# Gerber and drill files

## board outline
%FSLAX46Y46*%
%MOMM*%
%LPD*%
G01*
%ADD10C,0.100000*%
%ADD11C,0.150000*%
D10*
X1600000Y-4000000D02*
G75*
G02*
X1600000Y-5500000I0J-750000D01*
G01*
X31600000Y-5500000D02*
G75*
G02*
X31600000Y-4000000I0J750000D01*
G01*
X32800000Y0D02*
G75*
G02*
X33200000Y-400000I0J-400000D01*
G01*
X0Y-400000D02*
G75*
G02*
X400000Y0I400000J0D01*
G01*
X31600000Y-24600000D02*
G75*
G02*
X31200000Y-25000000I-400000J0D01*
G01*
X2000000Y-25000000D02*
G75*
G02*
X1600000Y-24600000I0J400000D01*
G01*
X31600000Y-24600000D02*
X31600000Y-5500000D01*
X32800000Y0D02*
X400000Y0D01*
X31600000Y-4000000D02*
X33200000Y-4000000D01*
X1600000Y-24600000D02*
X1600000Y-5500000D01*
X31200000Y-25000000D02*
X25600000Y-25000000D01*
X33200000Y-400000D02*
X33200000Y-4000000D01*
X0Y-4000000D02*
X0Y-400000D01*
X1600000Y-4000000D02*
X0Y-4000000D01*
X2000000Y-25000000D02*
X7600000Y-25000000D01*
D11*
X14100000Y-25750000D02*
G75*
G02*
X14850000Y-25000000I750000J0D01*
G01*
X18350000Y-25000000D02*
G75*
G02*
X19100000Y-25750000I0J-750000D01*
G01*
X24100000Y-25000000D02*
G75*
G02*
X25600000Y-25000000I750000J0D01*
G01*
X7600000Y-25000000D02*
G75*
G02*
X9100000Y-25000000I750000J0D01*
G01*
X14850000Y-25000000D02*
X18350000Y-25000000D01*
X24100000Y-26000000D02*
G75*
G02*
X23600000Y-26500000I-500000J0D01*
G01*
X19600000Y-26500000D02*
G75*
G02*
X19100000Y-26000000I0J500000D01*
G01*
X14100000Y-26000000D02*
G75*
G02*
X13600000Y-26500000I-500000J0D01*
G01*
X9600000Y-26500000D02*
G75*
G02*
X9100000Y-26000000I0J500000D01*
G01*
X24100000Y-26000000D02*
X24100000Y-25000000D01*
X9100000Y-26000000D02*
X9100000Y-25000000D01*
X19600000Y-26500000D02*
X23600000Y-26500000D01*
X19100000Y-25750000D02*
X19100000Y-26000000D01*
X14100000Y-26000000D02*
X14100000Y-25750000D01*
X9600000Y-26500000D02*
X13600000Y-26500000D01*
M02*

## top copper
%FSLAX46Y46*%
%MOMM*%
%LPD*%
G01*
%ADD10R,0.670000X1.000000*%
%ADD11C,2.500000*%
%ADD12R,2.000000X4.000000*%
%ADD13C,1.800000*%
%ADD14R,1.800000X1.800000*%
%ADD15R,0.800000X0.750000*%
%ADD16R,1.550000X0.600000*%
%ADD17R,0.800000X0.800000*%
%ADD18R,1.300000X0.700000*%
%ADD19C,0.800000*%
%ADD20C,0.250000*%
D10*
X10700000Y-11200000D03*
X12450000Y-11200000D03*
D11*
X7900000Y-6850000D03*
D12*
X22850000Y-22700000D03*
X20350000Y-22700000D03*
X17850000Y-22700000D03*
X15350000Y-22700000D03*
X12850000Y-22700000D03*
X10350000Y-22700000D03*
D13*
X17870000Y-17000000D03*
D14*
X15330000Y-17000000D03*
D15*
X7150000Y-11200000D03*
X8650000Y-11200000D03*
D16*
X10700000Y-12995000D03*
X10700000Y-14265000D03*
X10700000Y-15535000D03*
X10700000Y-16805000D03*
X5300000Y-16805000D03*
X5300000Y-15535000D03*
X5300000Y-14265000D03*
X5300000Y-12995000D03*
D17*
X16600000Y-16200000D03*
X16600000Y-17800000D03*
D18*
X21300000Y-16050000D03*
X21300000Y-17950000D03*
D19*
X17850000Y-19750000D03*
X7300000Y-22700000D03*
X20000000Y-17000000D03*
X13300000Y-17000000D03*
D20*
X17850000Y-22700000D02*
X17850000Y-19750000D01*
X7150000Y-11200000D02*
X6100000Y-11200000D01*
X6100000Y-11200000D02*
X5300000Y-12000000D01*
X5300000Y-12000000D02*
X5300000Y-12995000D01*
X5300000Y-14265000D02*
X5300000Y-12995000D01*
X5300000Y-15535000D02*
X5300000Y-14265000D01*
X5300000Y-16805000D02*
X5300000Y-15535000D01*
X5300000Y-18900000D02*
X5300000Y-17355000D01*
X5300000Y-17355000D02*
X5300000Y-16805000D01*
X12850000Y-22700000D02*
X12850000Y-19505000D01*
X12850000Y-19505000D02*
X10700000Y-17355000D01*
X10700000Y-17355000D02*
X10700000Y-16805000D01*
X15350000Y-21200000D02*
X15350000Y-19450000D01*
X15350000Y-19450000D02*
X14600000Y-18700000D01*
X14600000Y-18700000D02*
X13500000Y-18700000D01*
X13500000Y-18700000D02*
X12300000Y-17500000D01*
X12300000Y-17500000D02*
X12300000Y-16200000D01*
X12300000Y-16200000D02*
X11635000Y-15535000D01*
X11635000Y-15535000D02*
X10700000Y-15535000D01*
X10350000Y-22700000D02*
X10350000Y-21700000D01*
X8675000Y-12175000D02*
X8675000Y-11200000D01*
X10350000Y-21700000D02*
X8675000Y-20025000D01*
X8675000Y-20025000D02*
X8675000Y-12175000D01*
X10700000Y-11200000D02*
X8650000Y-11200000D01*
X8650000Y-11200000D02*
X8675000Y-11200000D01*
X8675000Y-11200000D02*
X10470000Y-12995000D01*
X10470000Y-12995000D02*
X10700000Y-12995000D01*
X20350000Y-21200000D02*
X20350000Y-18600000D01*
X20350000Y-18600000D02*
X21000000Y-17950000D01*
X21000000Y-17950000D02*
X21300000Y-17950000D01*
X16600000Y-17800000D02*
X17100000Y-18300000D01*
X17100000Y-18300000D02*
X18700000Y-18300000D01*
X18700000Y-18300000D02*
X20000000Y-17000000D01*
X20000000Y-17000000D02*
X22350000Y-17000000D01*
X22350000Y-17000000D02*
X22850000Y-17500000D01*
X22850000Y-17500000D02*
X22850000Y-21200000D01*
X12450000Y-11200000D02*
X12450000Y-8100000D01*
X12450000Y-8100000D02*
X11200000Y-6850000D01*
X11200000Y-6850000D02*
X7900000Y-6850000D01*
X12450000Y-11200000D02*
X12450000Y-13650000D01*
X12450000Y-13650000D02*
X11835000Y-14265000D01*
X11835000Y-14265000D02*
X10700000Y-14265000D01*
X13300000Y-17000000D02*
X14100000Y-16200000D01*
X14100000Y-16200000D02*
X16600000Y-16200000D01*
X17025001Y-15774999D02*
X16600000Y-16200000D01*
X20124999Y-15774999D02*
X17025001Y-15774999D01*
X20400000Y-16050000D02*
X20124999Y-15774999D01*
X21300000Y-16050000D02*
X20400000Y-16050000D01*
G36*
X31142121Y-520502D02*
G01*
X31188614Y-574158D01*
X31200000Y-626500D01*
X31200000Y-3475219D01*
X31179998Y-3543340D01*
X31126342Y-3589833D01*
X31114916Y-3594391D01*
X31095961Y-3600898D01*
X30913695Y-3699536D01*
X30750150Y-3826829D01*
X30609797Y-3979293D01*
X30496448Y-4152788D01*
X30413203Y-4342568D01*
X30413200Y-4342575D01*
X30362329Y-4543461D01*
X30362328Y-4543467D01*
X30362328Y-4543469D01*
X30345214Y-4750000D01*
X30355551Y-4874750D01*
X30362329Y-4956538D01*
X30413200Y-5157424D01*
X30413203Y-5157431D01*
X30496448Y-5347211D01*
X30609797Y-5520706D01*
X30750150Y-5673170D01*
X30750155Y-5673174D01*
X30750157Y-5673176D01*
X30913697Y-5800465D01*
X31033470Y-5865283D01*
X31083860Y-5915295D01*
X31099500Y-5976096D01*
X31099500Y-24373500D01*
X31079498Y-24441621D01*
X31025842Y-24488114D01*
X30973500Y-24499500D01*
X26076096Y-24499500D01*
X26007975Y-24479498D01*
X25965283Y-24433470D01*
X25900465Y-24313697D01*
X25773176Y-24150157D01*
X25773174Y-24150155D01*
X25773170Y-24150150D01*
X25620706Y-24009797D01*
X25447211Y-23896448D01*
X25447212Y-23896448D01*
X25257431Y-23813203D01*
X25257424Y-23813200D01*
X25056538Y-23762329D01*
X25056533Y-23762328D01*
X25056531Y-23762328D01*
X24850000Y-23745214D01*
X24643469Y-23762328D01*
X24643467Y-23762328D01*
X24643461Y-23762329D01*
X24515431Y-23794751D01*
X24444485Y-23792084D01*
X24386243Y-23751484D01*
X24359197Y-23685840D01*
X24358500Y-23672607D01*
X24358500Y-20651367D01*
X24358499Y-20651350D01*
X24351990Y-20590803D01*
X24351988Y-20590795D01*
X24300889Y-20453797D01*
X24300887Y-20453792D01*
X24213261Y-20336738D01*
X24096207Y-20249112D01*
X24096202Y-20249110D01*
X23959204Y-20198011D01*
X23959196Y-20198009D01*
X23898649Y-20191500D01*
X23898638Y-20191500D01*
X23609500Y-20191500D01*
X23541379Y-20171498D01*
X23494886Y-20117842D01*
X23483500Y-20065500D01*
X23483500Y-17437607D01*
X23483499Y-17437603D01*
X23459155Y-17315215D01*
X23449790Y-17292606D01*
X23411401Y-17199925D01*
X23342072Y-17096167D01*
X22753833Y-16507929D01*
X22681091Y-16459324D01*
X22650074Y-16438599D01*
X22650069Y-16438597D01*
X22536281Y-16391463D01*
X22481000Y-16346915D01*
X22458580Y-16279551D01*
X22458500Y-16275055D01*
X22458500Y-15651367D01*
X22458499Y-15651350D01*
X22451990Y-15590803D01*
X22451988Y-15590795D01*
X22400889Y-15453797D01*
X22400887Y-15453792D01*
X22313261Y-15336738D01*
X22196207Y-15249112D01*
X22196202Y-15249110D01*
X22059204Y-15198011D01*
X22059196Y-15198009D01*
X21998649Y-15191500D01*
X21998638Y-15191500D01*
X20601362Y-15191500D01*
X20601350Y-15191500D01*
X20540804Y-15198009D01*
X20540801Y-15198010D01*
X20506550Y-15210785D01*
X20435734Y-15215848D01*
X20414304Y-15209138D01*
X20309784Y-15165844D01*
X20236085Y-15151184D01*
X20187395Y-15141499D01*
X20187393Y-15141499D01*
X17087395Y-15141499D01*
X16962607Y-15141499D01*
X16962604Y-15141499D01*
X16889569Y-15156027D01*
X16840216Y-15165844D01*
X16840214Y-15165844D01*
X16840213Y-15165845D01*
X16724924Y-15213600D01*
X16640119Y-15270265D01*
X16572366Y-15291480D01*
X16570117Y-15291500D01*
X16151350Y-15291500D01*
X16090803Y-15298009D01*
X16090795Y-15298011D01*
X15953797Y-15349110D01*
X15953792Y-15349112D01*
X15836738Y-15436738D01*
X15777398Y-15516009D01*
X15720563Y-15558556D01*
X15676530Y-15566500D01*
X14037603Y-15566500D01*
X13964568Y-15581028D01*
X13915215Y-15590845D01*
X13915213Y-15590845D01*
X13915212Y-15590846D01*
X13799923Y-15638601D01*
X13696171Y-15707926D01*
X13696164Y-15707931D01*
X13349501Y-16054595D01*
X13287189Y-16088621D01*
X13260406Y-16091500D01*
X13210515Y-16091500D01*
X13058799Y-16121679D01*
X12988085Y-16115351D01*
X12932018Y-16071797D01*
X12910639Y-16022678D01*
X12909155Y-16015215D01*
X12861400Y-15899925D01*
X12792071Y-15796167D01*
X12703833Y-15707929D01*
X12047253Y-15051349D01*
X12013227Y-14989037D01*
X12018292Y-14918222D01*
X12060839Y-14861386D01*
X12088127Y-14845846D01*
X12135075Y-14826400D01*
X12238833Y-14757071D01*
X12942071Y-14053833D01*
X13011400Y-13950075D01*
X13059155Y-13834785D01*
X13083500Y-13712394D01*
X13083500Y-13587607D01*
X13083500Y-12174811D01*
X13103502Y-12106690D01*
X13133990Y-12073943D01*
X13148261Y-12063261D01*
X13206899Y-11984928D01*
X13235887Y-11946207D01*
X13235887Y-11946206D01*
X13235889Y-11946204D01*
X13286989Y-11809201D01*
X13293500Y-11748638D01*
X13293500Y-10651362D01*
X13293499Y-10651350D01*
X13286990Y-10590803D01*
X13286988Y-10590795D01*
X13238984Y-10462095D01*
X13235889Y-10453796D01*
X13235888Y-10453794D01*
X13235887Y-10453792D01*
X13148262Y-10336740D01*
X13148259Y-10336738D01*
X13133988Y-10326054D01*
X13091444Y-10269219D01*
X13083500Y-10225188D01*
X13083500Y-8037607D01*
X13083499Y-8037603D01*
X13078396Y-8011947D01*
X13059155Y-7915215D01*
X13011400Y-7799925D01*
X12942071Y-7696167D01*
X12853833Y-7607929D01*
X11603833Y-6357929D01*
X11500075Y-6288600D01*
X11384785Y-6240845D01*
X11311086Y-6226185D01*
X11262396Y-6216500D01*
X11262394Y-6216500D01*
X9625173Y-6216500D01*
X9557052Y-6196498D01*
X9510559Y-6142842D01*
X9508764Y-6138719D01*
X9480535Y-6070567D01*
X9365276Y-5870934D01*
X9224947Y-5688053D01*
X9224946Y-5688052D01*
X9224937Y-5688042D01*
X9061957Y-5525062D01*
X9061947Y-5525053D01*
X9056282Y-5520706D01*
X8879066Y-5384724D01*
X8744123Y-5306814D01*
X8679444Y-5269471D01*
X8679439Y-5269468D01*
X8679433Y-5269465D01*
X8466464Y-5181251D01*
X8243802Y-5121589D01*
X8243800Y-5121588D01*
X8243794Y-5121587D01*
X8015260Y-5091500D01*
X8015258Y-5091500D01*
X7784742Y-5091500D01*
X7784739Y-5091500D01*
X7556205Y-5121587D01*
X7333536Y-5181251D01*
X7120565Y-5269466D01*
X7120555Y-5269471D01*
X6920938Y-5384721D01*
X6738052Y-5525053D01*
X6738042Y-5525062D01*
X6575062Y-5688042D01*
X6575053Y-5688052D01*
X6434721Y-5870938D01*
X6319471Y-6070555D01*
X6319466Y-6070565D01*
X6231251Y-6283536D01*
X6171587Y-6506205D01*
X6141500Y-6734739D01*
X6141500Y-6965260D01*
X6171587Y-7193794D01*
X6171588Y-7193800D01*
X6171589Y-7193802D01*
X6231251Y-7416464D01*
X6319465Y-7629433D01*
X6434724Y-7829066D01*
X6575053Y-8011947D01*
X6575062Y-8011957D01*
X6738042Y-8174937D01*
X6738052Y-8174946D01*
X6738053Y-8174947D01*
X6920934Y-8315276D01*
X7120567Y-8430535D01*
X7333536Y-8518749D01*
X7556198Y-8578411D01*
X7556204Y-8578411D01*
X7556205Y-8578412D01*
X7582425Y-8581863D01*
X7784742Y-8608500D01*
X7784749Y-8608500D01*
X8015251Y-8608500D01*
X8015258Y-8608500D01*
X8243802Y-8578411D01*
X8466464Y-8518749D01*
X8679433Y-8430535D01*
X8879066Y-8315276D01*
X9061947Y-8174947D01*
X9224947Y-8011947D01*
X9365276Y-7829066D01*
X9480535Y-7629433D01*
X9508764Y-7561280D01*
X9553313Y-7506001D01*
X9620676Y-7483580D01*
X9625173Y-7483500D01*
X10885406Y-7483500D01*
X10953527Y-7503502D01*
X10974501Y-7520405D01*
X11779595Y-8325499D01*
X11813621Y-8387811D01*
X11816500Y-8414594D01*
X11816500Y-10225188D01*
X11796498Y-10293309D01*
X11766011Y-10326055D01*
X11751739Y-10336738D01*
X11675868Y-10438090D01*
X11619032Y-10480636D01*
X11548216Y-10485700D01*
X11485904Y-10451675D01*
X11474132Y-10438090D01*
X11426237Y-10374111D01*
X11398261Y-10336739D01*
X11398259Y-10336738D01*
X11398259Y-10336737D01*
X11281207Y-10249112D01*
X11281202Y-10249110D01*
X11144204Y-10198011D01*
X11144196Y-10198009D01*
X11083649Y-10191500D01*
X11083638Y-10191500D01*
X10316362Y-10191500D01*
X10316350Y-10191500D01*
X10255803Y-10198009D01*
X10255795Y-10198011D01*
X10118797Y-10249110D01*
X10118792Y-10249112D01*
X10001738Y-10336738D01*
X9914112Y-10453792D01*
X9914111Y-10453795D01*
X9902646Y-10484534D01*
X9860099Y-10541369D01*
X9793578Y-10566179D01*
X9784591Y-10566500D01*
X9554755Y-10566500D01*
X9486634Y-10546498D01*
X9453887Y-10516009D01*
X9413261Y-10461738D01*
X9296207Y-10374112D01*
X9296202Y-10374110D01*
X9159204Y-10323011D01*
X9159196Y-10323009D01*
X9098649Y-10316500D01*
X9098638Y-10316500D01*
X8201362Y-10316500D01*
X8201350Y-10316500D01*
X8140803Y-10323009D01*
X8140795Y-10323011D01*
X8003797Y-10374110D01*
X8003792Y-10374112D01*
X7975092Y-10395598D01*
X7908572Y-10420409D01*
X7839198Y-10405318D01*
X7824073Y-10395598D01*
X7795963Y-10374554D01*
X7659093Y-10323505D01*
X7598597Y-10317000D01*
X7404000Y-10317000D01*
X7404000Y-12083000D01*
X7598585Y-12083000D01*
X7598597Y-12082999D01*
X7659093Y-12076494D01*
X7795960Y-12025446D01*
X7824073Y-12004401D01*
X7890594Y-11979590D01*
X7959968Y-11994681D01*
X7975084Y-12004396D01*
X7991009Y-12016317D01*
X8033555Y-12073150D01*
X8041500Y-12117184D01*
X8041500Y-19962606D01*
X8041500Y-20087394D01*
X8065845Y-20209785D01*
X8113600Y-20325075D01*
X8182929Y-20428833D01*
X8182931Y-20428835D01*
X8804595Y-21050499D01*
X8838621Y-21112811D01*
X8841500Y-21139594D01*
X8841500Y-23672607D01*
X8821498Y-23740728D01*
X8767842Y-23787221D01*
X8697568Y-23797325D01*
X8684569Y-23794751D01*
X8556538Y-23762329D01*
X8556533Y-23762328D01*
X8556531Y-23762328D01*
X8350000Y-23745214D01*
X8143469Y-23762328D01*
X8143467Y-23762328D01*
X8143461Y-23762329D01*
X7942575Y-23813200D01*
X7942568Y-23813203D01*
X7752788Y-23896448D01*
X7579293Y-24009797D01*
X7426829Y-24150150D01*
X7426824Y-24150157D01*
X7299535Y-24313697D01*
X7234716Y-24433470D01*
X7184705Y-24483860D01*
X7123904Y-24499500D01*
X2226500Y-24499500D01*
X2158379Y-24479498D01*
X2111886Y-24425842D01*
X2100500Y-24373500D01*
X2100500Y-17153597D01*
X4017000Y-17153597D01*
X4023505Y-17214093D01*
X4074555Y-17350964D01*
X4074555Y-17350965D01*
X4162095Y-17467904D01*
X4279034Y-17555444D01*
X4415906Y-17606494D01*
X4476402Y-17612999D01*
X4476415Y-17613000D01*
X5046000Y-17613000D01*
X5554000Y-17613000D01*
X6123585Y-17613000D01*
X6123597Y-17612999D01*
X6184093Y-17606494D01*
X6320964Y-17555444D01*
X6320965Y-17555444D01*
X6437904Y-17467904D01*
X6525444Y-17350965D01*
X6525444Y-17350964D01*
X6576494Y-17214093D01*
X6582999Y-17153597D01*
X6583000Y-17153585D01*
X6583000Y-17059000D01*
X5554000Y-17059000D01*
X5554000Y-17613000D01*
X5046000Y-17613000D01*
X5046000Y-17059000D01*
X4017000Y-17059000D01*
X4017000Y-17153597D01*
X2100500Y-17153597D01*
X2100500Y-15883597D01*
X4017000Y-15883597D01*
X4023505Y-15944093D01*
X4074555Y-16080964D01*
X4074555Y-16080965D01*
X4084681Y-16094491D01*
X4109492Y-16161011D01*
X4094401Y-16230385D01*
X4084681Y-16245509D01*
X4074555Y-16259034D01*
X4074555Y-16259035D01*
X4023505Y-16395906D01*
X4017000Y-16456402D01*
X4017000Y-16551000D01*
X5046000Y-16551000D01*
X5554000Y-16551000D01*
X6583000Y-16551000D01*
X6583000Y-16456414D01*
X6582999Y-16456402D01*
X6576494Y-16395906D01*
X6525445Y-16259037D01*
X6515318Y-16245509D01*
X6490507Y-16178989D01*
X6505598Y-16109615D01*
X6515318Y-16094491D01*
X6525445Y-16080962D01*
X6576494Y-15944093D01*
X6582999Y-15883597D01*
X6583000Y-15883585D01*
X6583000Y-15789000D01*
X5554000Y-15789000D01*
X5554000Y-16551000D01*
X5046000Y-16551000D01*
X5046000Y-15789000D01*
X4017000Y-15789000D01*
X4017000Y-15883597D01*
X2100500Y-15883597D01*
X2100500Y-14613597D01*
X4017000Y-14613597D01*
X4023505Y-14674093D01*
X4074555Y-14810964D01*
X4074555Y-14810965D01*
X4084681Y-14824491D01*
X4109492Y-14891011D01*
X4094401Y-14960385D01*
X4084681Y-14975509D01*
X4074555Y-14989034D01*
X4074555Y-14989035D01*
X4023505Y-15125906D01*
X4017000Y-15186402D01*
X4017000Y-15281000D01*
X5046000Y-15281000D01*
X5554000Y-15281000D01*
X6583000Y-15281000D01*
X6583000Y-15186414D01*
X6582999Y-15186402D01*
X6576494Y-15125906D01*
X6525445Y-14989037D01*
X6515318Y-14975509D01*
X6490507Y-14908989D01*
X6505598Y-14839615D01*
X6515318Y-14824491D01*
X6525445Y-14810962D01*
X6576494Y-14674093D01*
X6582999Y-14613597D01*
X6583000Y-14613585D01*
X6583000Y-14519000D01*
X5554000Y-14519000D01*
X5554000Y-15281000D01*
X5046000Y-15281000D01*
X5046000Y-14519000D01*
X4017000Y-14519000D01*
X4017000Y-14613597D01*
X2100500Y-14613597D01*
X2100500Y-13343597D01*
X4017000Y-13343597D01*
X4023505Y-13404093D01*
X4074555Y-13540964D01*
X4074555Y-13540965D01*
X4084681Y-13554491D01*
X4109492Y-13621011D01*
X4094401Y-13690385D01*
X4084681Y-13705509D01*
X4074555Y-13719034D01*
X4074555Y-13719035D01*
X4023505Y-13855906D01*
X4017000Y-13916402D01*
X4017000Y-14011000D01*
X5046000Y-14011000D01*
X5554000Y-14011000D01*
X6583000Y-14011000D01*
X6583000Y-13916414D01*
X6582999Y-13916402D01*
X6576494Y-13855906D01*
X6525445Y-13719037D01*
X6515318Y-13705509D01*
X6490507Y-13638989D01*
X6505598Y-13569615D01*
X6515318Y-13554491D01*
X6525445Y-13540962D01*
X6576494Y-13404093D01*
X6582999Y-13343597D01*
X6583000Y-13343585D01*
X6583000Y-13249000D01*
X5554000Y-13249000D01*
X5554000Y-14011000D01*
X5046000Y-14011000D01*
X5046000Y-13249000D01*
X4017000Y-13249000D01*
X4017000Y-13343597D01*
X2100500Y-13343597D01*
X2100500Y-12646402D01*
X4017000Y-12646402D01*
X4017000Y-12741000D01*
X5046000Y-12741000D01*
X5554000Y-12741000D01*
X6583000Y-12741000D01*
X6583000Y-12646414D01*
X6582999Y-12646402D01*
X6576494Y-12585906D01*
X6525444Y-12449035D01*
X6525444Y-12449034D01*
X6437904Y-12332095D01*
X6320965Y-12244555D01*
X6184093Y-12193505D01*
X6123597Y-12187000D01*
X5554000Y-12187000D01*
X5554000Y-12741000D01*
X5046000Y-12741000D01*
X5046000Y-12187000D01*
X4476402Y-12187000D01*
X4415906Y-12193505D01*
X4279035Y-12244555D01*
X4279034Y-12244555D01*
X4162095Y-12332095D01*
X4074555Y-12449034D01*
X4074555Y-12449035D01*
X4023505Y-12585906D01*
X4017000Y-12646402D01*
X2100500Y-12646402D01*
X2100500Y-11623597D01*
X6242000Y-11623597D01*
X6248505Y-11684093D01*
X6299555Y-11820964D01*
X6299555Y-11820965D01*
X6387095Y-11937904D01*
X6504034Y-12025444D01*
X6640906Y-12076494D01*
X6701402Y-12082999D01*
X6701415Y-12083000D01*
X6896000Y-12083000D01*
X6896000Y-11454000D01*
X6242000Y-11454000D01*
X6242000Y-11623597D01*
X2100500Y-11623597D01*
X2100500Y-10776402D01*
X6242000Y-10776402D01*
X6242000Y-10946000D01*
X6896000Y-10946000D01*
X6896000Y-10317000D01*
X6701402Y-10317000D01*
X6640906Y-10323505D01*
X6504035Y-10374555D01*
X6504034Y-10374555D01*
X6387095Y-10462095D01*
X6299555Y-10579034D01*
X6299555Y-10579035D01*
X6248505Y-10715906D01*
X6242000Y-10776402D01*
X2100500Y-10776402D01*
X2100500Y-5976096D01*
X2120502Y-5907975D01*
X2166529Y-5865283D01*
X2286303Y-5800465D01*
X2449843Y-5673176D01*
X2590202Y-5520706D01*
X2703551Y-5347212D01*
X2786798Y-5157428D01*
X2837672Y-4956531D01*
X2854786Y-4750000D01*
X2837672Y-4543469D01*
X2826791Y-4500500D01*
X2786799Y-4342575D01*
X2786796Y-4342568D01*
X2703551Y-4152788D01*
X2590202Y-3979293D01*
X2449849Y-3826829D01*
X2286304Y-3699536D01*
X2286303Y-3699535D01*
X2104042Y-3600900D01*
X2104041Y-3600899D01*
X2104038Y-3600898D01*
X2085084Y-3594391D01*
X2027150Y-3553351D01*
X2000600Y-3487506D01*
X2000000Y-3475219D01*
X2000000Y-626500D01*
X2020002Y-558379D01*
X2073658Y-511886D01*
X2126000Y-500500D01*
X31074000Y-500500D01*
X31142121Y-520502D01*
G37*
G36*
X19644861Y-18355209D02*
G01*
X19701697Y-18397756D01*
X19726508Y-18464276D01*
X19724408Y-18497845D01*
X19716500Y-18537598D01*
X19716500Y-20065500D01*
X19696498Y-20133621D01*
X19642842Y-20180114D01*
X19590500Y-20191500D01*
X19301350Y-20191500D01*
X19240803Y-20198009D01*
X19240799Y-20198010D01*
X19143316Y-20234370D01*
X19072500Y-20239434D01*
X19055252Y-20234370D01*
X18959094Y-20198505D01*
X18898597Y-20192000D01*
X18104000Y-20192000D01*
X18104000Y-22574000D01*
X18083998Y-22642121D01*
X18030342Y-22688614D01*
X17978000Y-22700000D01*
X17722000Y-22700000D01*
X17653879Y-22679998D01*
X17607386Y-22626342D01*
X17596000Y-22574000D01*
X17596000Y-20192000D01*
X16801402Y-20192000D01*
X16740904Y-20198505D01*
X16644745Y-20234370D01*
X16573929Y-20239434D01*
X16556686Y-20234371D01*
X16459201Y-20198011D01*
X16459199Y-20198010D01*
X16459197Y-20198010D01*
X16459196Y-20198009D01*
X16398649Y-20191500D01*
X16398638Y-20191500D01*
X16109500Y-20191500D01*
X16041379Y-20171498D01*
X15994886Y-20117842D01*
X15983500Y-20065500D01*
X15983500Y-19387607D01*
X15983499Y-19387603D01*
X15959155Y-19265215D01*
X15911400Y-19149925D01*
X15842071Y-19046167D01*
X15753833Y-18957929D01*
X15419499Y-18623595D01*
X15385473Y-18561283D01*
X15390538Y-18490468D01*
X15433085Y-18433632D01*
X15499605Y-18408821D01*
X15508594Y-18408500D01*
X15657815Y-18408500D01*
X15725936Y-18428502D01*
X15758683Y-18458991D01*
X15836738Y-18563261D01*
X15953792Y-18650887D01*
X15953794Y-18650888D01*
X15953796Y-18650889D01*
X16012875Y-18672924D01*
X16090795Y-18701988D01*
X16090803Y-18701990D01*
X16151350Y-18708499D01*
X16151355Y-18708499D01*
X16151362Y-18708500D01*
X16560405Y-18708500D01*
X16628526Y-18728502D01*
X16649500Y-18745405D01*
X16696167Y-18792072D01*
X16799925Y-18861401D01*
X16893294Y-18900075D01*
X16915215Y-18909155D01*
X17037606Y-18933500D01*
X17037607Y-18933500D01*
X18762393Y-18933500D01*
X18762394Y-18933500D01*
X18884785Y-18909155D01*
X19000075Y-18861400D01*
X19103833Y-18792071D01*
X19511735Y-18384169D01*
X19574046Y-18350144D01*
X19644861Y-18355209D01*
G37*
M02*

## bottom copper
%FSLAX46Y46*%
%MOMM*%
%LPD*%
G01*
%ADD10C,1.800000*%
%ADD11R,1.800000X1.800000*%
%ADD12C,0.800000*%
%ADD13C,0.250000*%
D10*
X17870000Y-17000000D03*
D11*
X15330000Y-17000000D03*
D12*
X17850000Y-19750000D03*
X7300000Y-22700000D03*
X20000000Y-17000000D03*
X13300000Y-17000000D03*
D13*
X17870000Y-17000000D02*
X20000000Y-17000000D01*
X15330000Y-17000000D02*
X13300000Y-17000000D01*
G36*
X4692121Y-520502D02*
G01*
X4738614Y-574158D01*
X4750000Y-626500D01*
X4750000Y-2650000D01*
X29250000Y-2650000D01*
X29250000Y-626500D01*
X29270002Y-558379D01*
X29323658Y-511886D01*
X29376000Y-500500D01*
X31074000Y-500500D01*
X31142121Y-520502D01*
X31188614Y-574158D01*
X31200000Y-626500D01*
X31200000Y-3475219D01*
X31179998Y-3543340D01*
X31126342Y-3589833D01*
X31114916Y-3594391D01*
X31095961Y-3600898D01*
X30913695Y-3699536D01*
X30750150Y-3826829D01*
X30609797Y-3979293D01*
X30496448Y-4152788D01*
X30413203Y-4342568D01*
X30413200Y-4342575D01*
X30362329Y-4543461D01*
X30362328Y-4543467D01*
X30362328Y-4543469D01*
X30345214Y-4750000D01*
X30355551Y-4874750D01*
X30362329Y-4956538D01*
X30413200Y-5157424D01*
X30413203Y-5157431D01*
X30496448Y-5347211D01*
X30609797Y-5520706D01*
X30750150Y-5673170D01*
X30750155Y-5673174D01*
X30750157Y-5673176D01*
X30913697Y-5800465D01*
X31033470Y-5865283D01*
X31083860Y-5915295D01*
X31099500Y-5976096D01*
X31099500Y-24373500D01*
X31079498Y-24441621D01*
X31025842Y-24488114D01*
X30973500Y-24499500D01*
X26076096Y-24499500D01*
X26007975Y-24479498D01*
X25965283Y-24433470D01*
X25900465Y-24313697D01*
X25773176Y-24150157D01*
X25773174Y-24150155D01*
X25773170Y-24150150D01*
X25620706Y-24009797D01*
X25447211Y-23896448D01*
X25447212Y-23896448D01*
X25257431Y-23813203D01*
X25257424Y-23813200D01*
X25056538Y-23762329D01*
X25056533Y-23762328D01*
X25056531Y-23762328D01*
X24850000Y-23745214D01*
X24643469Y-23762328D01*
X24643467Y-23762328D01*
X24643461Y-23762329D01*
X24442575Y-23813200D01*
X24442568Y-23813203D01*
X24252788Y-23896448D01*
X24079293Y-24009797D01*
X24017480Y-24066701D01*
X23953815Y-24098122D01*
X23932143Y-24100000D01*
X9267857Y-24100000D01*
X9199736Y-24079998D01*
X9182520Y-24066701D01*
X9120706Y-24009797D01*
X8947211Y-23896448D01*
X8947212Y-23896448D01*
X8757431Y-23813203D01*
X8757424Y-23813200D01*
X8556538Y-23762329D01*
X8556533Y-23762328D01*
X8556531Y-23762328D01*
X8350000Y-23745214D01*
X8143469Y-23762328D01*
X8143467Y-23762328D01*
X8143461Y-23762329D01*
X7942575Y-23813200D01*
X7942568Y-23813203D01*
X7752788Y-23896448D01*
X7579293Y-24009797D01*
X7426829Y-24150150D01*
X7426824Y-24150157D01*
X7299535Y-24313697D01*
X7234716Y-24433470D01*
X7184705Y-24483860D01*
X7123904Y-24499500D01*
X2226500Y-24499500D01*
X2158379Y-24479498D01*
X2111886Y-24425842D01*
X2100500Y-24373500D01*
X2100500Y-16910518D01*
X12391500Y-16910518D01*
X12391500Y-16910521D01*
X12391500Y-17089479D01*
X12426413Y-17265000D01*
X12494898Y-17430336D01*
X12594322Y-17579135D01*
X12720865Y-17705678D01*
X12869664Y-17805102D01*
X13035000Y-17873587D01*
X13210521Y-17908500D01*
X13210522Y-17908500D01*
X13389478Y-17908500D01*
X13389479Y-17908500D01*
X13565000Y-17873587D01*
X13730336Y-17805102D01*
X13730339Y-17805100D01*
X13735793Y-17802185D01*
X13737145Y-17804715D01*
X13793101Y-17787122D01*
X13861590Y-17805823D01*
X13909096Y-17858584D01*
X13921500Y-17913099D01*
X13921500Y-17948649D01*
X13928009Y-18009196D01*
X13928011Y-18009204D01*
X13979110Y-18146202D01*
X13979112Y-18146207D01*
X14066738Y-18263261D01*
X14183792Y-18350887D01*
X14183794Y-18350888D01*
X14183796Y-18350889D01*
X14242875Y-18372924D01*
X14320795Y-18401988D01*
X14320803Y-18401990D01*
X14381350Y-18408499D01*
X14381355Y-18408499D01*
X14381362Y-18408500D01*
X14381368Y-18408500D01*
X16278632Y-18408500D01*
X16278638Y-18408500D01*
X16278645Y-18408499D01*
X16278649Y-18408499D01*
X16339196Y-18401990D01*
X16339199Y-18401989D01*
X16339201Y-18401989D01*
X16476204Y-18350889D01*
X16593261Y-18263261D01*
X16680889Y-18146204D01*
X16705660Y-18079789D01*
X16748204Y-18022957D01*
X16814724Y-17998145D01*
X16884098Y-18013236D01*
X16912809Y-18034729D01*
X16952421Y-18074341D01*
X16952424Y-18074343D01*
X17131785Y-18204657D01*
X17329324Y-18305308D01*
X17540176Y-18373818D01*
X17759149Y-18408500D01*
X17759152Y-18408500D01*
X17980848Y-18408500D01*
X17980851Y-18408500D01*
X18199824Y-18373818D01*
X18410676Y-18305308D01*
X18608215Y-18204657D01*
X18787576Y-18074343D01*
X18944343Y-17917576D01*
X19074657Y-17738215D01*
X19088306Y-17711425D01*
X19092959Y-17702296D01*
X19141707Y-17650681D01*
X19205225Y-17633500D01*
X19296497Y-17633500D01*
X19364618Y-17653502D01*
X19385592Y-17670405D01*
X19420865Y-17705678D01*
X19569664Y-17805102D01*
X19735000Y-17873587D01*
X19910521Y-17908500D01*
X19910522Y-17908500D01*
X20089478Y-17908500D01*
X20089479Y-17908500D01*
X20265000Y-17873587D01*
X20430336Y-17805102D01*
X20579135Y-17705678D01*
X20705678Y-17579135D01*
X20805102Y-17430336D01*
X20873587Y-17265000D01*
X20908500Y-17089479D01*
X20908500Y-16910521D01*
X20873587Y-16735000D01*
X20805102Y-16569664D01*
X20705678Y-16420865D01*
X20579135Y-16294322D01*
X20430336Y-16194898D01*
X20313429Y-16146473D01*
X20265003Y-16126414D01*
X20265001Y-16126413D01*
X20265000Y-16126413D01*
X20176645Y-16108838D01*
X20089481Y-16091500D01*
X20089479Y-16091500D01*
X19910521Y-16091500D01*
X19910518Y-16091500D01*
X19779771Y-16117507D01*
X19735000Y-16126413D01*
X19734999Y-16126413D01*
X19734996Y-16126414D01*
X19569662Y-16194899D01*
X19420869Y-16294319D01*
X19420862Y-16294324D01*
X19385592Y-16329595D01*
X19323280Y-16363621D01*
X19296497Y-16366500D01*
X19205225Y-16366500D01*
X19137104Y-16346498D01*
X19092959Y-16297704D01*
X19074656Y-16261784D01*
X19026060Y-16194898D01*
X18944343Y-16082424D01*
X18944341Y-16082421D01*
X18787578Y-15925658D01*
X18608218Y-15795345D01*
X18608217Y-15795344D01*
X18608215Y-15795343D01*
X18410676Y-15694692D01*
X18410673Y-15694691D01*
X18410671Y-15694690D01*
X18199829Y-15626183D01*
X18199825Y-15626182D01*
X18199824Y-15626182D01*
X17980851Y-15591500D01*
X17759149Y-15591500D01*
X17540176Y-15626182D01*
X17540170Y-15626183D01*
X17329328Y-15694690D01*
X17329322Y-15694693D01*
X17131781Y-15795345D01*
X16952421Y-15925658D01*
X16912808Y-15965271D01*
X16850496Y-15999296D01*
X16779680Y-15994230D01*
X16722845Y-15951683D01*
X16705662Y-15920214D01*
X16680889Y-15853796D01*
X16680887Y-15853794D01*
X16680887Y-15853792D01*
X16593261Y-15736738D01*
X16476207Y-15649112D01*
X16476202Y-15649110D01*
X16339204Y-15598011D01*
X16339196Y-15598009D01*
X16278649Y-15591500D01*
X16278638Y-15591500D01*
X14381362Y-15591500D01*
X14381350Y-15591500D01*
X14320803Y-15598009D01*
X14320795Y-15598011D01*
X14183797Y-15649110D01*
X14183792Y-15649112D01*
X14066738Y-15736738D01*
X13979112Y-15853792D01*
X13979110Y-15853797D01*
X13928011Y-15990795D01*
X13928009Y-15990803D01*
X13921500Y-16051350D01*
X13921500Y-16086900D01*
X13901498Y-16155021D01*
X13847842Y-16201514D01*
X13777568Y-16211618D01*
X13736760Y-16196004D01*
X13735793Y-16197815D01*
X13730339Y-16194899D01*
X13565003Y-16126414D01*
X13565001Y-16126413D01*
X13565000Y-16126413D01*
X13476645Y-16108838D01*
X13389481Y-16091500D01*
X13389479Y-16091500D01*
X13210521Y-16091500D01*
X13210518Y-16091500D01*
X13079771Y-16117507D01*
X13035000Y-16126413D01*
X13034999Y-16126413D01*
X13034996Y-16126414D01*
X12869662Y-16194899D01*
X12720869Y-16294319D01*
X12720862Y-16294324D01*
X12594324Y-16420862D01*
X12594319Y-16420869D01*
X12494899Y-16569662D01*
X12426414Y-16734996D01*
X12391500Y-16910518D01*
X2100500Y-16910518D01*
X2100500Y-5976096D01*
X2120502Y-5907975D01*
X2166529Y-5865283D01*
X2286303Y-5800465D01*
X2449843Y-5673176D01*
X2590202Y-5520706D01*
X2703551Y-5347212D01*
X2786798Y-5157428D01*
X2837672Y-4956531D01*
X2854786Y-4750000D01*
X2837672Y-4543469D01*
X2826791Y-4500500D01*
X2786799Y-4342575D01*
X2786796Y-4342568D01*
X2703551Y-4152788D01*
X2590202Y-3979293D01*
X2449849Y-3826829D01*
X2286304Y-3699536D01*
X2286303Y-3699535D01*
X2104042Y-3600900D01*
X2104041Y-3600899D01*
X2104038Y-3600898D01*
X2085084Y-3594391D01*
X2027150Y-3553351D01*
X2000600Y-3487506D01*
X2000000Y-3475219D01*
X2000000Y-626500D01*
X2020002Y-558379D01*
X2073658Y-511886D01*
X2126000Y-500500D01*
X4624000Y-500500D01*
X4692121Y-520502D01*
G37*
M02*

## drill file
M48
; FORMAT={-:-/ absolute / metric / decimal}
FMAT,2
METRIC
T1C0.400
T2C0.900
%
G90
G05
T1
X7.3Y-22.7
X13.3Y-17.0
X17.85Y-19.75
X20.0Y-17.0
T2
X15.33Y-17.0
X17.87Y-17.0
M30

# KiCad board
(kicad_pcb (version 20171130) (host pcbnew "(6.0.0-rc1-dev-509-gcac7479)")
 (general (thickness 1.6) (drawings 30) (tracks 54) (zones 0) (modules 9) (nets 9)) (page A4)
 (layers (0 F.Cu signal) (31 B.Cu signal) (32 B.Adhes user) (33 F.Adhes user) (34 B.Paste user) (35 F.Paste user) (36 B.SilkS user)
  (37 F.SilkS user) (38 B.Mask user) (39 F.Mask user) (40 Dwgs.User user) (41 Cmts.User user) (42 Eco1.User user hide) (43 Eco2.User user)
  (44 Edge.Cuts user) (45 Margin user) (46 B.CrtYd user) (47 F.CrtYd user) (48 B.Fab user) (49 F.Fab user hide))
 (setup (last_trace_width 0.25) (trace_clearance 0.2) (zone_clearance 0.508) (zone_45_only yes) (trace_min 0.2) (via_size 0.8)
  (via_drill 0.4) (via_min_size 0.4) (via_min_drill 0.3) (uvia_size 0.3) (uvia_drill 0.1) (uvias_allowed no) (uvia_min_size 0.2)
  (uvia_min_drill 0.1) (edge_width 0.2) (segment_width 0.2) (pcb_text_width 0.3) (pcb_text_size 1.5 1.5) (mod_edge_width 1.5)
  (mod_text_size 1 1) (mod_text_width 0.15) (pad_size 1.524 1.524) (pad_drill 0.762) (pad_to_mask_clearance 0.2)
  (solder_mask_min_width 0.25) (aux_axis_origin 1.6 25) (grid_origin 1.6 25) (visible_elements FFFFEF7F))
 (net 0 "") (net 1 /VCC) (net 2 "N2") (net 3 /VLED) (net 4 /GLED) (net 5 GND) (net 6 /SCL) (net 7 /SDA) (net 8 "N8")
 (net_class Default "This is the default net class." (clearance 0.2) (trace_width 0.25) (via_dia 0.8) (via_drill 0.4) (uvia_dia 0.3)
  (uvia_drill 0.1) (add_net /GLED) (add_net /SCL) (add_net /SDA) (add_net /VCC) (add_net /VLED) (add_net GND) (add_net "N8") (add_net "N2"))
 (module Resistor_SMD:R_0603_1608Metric (layer F.Cu) (at 11.575 11.2)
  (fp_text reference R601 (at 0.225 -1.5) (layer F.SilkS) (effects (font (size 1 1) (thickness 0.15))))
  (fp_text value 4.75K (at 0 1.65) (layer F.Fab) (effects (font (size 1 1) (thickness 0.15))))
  (pad 1 smd rect (at -0.875 0) (size 0.67 1) (layers F.Cu F.Paste F.Mask) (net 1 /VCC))
  (pad 2 smd rect (at 0.875 0) (size 0.67 1) (layers F.Cu F.Paste F.Mask) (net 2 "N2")))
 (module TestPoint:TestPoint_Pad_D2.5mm (layer F.Cu) (at 7.9 6.85)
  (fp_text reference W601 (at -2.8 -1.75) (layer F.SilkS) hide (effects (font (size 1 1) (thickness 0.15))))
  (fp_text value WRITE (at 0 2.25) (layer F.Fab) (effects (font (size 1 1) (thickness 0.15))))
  (pad 1 smd circle (at 0 0) (size 2.5 2.5) (layers F.Cu F.Mask) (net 2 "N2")))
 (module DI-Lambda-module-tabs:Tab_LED (layer F.Cu) (at 16.6 25)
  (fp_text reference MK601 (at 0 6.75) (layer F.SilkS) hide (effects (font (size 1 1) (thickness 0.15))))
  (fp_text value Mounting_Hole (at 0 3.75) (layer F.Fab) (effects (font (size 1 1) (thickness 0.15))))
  (fp_arc (start -1.75 0.75) (end -1.75 0) (angle -90) (layer Edge.Cuts) (width 0.15))
  (fp_arc (start 1.75 0.75) (end 2.5 0.75) (angle -90) (layer Edge.Cuts) (width 0.15))
  (fp_arc (start 8.25 0) (end 9 0) (angle -180) (layer Edge.Cuts) (width 0.15))
  (fp_arc (start -8.25 0) (end -7.5 0) (angle -180) (layer Edge.Cuts) (width 0.15))
  (fp_line (start -1.75 0) (end 1.75 0) (layer Edge.Cuts) (width 0.15))
  (fp_arc (start 7 1) (end 7 1.5) (angle -90) (layer Edge.Cuts) (width 0.15))
  (fp_arc (start 3 1) (end 2.5 1) (angle -90) (layer Edge.Cuts) (width 0.15))
  (fp_arc (start -3 1) (end -3 1.5) (angle -90) (layer Edge.Cuts) (width 0.15))
  (fp_arc (start -7 1) (end -7.5 1) (angle -90) (layer Edge.Cuts) (width 0.15))
  (fp_line (start 7.5 1) (end 7.5 0) (layer Edge.Cuts) (width 0.15))
  (fp_line (start -7.5 1) (end -7.5 0) (layer Edge.Cuts) (width 0.15))
  (fp_line (start 3 1.5) (end 7 1.5) (layer Edge.Cuts) (width 0.15))
  (fp_line (start 2.5 0.75) (end 2.5 1) (layer Edge.Cuts) (width 0.15))
  (fp_line (start -2.5 1) (end -2.5 0.75) (layer Edge.Cuts) (width 0.15))
  (fp_line (start -7 1.5) (end -3 1.5) (layer Edge.Cuts) (width 0.15)))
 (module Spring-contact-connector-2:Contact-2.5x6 (layer F.Cu) (at 16.6 23.7)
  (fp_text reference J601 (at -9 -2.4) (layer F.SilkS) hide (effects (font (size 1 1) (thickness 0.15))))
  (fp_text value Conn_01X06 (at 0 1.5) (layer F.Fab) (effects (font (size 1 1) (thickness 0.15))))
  (pad 6 smd rect (at 6.25 -1) (size 2 4) (layers F.Cu F.Paste F.Mask) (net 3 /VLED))
  (pad 5 smd rect (at 3.75 -1) (size 2 4) (layers F.Cu F.Paste F.Mask) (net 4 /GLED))
  (pad 4 smd rect (at 1.25 -1) (size 2 4) (layers F.Cu F.Paste F.Mask) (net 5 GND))
  (pad 3 smd rect (at -1.25 -1) (size 2 4) (layers F.Cu F.Paste F.Mask) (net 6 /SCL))
  (pad 2 smd rect (at -3.75 -1) (size 2 4) (layers F.Cu F.Paste F.Mask) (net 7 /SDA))
  (pad 1 smd rect (at -6.25 -1) (size 2 4) (layers F.Cu F.Paste F.Mask) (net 1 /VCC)))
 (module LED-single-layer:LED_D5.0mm (layer F.Cu) (at 15.33 17)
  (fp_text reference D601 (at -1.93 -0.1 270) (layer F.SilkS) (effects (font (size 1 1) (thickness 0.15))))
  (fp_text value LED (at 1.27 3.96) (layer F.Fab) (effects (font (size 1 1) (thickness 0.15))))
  (pad 2 thru_hole circle (at 2.54 0) (size 1.8 1.8) (drill 0.9) (layers B.Cu B.Mask) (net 3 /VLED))
  (pad 1 thru_hole rect (at 0 0) (size 1.8 1.8) (drill 0.9) (layers B.Cu B.Mask) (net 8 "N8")))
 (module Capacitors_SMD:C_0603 (layer F.Cu) (at 7.9 11.2 180)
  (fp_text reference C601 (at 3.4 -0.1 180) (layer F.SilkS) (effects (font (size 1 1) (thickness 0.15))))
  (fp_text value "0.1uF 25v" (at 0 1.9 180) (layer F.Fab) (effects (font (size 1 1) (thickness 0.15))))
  (pad 2 smd rect (at 0.75 0 180) (size 0.8 0.75) (layers F.Cu F.Paste F.Mask) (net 5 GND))
  (pad 1 smd rect (at -0.75 0 180) (size 0.8 0.75) (layers F.Cu F.Paste F.Mask) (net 1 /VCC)))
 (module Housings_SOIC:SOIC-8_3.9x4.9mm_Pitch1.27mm (layer F.Cu) (at 8 14.9)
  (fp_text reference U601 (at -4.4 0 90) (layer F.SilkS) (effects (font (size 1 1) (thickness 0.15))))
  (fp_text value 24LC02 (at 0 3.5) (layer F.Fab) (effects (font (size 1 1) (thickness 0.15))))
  (pad 8 smd rect (at 2.7 -1.905) (size 1.55 0.6) (layers F.Cu F.Paste F.Mask) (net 1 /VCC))
  (pad 7 smd rect (at 2.7 -0.635) (size 1.55 0.6) (layers F.Cu F.Paste F.Mask) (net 2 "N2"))
  (pad 6 smd rect (at 2.7 0.635) (size 1.55 0.6) (layers F.Cu F.Paste F.Mask) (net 6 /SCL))
  (pad 5 smd rect (at 2.7 1.905) (size 1.55 0.6) (layers F.Cu F.Paste F.Mask) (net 7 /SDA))
  (pad 4 smd rect (at -2.7 1.905) (size 1.55 0.6) (layers F.Cu F.Paste F.Mask) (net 5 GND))
  (pad 3 smd rect (at -2.7 0.635) (size 1.55 0.6) (layers F.Cu F.Paste F.Mask) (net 5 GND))
  (pad 2 smd rect (at -2.7 -0.635) (size 1.55 0.6) (layers F.Cu F.Paste F.Mask) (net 5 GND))
  (pad 1 smd rect (at -2.7 -1.905) (size 1.55 0.6) (layers F.Cu F.Paste F.Mask) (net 5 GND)))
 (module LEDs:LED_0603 (layer F.Cu) (at 16.6 17 270)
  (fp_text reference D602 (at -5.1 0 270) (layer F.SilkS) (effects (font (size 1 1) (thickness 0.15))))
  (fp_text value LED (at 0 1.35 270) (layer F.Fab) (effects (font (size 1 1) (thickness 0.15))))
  (pad 1 smd rect (at -0.8 0 90) (size 0.8 0.8) (layers F.Cu F.Paste F.Mask) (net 8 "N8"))
  (pad 2 smd rect (at 0.8 0 90) (size 0.8 0.8) (layers F.Cu F.Paste F.Mask) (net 3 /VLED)))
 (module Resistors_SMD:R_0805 (layer F.Cu) (at 21.3 17 90)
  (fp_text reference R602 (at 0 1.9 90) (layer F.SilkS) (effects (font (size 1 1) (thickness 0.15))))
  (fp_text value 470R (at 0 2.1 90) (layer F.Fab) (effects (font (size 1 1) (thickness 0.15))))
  (pad 2 smd rect (at 0.95 0 90) (size 0.7 1.3) (layers F.Cu F.Paste F.Mask) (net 8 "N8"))
  (pad 1 smd rect (at -0.95 0 90) (size 0.7 1.3) (layers F.Cu F.Paste F.Mask) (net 4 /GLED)))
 (gr_arc (start 1.6 4.75) (end 1.6 4) (angle 180) (layer Edge.Cuts) (width 0.1))
 (gr_arc (start 31.6 4.75) (end 31.6 5.5) (angle 180) (layer Edge.Cuts) (width 0.1))
 (gr_arc (start 32.8 0.4) (end 32.8 0) (angle 90) (layer Edge.Cuts) (width 0.1))
 (gr_arc (start 0.4 0.4) (end 0 0.4) (angle 90) (layer Edge.Cuts) (width 0.1))
 (gr_arc (start 31.2 24.6) (end 31.6 24.6) (angle 90) (layer Edge.Cuts) (width 0.1))
 (gr_arc (start 2 24.6) (end 2 25) (angle 90) (layer Edge.Cuts) (width 0.1))
 (gr_line (start 31.6 24.6) (end 31.6 5.5) (layer Edge.Cuts) (width 0.1))
 (gr_line (start 32.8 0) (end 0.4 0) (layer Edge.Cuts) (width 0.1))
 (gr_line (start 31.6 4) (end 33.2 4) (layer Edge.Cuts) (width 0.1))
 (gr_line (start 1.6 24.6) (end 1.6 5.5) (layer Edge.Cuts) (width 0.1))
 (gr_line (start 31.2 25) (end 25.6 25) (layer Edge.Cuts) (width 0.1))
 (gr_line (start 33.2 0.4) (end 33.2 4) (layer Edge.Cuts) (width 0.1))
 (gr_line (start 0 4) (end 0 0.4) (layer Edge.Cuts) (width 0.1))
 (gr_line (start 1.6 4) (end 0 4) (layer Edge.Cuts) (width 0.1))
 (gr_line (start 2 25) (end 7.6 25) (layer Edge.Cuts) (width 0.1))
 (segment (start 17.85 22.7) (end 17.85 19.75) (width 0.25) (layer F.Cu) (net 5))
 (via (at 17.85 19.75) (size 0.8) (drill 0.4) (layers F.Cu B.Cu) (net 5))
 (via (at 7.3 22.7) (size 0.8) (drill 0.4) (layers F.Cu B.Cu) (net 5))
 (segment (start 7.15 11.2) (end 6.1 11.2) (width 0.25) (layer F.Cu) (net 5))
 (segment (start 6.1 11.2) (end 5.3 12) (width 0.25) (layer F.Cu) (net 5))
 (segment (start 5.3 12) (end 5.3 12.995) (width 0.25) (layer F.Cu) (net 5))
 (segment (start 5.3 14.265) (end 5.3 12.995) (width 0.25) (layer F.Cu) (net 5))
 (segment (start 5.3 15.535) (end 5.3 14.265) (width 0.25) (layer F.Cu) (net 5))
 (segment (start 5.3 16.805) (end 5.3 15.535) (width 0.25) (layer F.Cu) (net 5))
 (segment (start 5.3 18.9) (end 5.3 17.355) (width 0.25) (layer F.Cu) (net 5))
 (segment (start 5.3 17.355) (end 5.3 16.805) (width 0.25) (layer F.Cu) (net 5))
 (segment (start 12.85 22.7) (end 12.85 19.505) (width 0.25) (layer F.Cu) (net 7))
 (segment (start 12.85 19.505) (end 10.7 17.355) (width 0.25) (layer F.Cu) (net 7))
 (segment (start 10.7 17.355) (end 10.7 16.805) (width 0.25) (layer F.Cu) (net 7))
 (segment (start 15.35 21.2) (end 15.35 19.45) (width 0.25) (layer F.Cu) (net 6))
 (segment (start 15.35 19.45) (end 14.6 18.7) (width 0.25) (layer F.Cu) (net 6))
 (segment (start 14.6 18.7) (end 13.5 18.7) (width 0.25) (layer F.Cu) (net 6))
 (segment (start 13.5 18.7) (end 12.3 17.5) (width 0.25) (layer F.Cu) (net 6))
 (segment (start 12.3 17.5) (end 12.3 16.2) (width 0.25) (layer F.Cu) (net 6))
 (segment (start 12.3 16.2) (end 11.635 15.535) (width 0.25) (layer F.Cu) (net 6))
 (segment (start 11.635 15.535) (end 10.7 15.535) (width 0.25) (layer F.Cu) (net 6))
 (segment (start 10.35 22.7) (end 10.35 21.7) (width 0.25) (layer F.Cu) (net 1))
 (segment (start 8.675 12.175) (end 8.675 11.2) (width 0.25) (layer F.Cu) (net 1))
 (segment (start 10.35 21.7) (end 8.675 20.025) (width 0.25) (layer F.Cu) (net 1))
 (segment (start 8.675 20.025) (end 8.675 12.175) (width 0.25) (layer F.Cu) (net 1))
 (segment (start 10.7 11.2) (end 8.65 11.2) (width 0.25) (layer F.Cu) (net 1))
 (segment (start 8.65 11.2) (end 8.675 11.2) (width 0.25) (layer F.Cu) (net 1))
 (segment (start 8.675 11.2) (end 10.47 12.995) (width 0.25) (layer F.Cu) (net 1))
 (segment (start 10.47 12.995) (end 10.7 12.995) (width 0.25) (layer F.Cu) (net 1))
 (segment (start 20.35 21.2) (end 20.35 18.6) (width 0.25) (layer F.Cu) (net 4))
 (segment (start 20.35 18.6) (end 21 17.95) (width 0.25) (layer F.Cu) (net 4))
 (segment (start 21 17.95) (end 21.3 17.95) (width 0.25) (layer F.Cu) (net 4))
 (segment (start 16.6 17.8) (end 17.1 18.3) (width 0.25) (layer F.Cu) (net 3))
 (segment (start 17.1 18.3) (end 18.7 18.3) (width 0.25) (layer F.Cu) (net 3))
 (segment (start 18.7 18.3) (end 20 17) (width 0.25) (layer F.Cu) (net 3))
 (segment (start 20 17) (end 22.35 17) (width 0.25) (layer F.Cu) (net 3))
 (segment (start 22.35 17) (end 22.85 17.5) (width 0.25) (layer F.Cu) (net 3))
 (segment (start 22.85 17.5) (end 22.85 21.2) (width 0.25) (layer F.Cu) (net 3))
 (segment (start 17.87 17) (end 20 17) (width 0.25) (layer B.Cu) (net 3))
 (via (at 20 17) (size 0.8) (drill 0.4) (layers F.Cu B.Cu) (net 3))
 (segment (start 12.45 11.2) (end 12.45 8.1) (width 0.25) (layer F.Cu) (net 2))
 (segment (start 12.45 8.1) (end 11.2 6.85) (width 0.25) (layer F.Cu) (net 2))
 (segment (start 11.2 6.85) (end 7.9 6.85) (width 0.25) (layer F.Cu) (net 2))
 (segment (start 12.45 11.2) (end 12.45 13.65) (width 0.25) (layer F.Cu) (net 2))
 (segment (start 12.45 13.65) (end 11.835 14.265) (width 0.25) (layer F.Cu) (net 2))
 (segment (start 11.835 14.265) (end 10.7 14.265) (width 0.25) (layer F.Cu) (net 2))
 (segment (start 13.3 17) (end 14.1 16.2) (width 0.25) (layer F.Cu) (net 8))
 (segment (start 14.1 16.2) (end 16.6 16.2) (width 0.25) (layer F.Cu) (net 8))
 (segment (start 17.025001 15.774999) (end 16.6 16.2) (width 0.25) (layer F.Cu) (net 8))
 (segment (start 20.124999 15.774999) (end 17.025001 15.774999) (width 0.25) (layer F.Cu) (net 8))
 (segment (start 20.4 16.05) (end 20.124999 15.774999) (width 0.25) (layer F.Cu) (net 8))
 (segment (start 21.3 16.05) (end 20.4 16.05) (width 0.25) (layer F.Cu) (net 8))
 (segment (start 15.33 17) (end 13.3 17) (width 0.25) (layer B.Cu) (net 8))
 (via (at 13.3 17) (size 0.8) (drill 0.4) (layers F.Cu B.Cu) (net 8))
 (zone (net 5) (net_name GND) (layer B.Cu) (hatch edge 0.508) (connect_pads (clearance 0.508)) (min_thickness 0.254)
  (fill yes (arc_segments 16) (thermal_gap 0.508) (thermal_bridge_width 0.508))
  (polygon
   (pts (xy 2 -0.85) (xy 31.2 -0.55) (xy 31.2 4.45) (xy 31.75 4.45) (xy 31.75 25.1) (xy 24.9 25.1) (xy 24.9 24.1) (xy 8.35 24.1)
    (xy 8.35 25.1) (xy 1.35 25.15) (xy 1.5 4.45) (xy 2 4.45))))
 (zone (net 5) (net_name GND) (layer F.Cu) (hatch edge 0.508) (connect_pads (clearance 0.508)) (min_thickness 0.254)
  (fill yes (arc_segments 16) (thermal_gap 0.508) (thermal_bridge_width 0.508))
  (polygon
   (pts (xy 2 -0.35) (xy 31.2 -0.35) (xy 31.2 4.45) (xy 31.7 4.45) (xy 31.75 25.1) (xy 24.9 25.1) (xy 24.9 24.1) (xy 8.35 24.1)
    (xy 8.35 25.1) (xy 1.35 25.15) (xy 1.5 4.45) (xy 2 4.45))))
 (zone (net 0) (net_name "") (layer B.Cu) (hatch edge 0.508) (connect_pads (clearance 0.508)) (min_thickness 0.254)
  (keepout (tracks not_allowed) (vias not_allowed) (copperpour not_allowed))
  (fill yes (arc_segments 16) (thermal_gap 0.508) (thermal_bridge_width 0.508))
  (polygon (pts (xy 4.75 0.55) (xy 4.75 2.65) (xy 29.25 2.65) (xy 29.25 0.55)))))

